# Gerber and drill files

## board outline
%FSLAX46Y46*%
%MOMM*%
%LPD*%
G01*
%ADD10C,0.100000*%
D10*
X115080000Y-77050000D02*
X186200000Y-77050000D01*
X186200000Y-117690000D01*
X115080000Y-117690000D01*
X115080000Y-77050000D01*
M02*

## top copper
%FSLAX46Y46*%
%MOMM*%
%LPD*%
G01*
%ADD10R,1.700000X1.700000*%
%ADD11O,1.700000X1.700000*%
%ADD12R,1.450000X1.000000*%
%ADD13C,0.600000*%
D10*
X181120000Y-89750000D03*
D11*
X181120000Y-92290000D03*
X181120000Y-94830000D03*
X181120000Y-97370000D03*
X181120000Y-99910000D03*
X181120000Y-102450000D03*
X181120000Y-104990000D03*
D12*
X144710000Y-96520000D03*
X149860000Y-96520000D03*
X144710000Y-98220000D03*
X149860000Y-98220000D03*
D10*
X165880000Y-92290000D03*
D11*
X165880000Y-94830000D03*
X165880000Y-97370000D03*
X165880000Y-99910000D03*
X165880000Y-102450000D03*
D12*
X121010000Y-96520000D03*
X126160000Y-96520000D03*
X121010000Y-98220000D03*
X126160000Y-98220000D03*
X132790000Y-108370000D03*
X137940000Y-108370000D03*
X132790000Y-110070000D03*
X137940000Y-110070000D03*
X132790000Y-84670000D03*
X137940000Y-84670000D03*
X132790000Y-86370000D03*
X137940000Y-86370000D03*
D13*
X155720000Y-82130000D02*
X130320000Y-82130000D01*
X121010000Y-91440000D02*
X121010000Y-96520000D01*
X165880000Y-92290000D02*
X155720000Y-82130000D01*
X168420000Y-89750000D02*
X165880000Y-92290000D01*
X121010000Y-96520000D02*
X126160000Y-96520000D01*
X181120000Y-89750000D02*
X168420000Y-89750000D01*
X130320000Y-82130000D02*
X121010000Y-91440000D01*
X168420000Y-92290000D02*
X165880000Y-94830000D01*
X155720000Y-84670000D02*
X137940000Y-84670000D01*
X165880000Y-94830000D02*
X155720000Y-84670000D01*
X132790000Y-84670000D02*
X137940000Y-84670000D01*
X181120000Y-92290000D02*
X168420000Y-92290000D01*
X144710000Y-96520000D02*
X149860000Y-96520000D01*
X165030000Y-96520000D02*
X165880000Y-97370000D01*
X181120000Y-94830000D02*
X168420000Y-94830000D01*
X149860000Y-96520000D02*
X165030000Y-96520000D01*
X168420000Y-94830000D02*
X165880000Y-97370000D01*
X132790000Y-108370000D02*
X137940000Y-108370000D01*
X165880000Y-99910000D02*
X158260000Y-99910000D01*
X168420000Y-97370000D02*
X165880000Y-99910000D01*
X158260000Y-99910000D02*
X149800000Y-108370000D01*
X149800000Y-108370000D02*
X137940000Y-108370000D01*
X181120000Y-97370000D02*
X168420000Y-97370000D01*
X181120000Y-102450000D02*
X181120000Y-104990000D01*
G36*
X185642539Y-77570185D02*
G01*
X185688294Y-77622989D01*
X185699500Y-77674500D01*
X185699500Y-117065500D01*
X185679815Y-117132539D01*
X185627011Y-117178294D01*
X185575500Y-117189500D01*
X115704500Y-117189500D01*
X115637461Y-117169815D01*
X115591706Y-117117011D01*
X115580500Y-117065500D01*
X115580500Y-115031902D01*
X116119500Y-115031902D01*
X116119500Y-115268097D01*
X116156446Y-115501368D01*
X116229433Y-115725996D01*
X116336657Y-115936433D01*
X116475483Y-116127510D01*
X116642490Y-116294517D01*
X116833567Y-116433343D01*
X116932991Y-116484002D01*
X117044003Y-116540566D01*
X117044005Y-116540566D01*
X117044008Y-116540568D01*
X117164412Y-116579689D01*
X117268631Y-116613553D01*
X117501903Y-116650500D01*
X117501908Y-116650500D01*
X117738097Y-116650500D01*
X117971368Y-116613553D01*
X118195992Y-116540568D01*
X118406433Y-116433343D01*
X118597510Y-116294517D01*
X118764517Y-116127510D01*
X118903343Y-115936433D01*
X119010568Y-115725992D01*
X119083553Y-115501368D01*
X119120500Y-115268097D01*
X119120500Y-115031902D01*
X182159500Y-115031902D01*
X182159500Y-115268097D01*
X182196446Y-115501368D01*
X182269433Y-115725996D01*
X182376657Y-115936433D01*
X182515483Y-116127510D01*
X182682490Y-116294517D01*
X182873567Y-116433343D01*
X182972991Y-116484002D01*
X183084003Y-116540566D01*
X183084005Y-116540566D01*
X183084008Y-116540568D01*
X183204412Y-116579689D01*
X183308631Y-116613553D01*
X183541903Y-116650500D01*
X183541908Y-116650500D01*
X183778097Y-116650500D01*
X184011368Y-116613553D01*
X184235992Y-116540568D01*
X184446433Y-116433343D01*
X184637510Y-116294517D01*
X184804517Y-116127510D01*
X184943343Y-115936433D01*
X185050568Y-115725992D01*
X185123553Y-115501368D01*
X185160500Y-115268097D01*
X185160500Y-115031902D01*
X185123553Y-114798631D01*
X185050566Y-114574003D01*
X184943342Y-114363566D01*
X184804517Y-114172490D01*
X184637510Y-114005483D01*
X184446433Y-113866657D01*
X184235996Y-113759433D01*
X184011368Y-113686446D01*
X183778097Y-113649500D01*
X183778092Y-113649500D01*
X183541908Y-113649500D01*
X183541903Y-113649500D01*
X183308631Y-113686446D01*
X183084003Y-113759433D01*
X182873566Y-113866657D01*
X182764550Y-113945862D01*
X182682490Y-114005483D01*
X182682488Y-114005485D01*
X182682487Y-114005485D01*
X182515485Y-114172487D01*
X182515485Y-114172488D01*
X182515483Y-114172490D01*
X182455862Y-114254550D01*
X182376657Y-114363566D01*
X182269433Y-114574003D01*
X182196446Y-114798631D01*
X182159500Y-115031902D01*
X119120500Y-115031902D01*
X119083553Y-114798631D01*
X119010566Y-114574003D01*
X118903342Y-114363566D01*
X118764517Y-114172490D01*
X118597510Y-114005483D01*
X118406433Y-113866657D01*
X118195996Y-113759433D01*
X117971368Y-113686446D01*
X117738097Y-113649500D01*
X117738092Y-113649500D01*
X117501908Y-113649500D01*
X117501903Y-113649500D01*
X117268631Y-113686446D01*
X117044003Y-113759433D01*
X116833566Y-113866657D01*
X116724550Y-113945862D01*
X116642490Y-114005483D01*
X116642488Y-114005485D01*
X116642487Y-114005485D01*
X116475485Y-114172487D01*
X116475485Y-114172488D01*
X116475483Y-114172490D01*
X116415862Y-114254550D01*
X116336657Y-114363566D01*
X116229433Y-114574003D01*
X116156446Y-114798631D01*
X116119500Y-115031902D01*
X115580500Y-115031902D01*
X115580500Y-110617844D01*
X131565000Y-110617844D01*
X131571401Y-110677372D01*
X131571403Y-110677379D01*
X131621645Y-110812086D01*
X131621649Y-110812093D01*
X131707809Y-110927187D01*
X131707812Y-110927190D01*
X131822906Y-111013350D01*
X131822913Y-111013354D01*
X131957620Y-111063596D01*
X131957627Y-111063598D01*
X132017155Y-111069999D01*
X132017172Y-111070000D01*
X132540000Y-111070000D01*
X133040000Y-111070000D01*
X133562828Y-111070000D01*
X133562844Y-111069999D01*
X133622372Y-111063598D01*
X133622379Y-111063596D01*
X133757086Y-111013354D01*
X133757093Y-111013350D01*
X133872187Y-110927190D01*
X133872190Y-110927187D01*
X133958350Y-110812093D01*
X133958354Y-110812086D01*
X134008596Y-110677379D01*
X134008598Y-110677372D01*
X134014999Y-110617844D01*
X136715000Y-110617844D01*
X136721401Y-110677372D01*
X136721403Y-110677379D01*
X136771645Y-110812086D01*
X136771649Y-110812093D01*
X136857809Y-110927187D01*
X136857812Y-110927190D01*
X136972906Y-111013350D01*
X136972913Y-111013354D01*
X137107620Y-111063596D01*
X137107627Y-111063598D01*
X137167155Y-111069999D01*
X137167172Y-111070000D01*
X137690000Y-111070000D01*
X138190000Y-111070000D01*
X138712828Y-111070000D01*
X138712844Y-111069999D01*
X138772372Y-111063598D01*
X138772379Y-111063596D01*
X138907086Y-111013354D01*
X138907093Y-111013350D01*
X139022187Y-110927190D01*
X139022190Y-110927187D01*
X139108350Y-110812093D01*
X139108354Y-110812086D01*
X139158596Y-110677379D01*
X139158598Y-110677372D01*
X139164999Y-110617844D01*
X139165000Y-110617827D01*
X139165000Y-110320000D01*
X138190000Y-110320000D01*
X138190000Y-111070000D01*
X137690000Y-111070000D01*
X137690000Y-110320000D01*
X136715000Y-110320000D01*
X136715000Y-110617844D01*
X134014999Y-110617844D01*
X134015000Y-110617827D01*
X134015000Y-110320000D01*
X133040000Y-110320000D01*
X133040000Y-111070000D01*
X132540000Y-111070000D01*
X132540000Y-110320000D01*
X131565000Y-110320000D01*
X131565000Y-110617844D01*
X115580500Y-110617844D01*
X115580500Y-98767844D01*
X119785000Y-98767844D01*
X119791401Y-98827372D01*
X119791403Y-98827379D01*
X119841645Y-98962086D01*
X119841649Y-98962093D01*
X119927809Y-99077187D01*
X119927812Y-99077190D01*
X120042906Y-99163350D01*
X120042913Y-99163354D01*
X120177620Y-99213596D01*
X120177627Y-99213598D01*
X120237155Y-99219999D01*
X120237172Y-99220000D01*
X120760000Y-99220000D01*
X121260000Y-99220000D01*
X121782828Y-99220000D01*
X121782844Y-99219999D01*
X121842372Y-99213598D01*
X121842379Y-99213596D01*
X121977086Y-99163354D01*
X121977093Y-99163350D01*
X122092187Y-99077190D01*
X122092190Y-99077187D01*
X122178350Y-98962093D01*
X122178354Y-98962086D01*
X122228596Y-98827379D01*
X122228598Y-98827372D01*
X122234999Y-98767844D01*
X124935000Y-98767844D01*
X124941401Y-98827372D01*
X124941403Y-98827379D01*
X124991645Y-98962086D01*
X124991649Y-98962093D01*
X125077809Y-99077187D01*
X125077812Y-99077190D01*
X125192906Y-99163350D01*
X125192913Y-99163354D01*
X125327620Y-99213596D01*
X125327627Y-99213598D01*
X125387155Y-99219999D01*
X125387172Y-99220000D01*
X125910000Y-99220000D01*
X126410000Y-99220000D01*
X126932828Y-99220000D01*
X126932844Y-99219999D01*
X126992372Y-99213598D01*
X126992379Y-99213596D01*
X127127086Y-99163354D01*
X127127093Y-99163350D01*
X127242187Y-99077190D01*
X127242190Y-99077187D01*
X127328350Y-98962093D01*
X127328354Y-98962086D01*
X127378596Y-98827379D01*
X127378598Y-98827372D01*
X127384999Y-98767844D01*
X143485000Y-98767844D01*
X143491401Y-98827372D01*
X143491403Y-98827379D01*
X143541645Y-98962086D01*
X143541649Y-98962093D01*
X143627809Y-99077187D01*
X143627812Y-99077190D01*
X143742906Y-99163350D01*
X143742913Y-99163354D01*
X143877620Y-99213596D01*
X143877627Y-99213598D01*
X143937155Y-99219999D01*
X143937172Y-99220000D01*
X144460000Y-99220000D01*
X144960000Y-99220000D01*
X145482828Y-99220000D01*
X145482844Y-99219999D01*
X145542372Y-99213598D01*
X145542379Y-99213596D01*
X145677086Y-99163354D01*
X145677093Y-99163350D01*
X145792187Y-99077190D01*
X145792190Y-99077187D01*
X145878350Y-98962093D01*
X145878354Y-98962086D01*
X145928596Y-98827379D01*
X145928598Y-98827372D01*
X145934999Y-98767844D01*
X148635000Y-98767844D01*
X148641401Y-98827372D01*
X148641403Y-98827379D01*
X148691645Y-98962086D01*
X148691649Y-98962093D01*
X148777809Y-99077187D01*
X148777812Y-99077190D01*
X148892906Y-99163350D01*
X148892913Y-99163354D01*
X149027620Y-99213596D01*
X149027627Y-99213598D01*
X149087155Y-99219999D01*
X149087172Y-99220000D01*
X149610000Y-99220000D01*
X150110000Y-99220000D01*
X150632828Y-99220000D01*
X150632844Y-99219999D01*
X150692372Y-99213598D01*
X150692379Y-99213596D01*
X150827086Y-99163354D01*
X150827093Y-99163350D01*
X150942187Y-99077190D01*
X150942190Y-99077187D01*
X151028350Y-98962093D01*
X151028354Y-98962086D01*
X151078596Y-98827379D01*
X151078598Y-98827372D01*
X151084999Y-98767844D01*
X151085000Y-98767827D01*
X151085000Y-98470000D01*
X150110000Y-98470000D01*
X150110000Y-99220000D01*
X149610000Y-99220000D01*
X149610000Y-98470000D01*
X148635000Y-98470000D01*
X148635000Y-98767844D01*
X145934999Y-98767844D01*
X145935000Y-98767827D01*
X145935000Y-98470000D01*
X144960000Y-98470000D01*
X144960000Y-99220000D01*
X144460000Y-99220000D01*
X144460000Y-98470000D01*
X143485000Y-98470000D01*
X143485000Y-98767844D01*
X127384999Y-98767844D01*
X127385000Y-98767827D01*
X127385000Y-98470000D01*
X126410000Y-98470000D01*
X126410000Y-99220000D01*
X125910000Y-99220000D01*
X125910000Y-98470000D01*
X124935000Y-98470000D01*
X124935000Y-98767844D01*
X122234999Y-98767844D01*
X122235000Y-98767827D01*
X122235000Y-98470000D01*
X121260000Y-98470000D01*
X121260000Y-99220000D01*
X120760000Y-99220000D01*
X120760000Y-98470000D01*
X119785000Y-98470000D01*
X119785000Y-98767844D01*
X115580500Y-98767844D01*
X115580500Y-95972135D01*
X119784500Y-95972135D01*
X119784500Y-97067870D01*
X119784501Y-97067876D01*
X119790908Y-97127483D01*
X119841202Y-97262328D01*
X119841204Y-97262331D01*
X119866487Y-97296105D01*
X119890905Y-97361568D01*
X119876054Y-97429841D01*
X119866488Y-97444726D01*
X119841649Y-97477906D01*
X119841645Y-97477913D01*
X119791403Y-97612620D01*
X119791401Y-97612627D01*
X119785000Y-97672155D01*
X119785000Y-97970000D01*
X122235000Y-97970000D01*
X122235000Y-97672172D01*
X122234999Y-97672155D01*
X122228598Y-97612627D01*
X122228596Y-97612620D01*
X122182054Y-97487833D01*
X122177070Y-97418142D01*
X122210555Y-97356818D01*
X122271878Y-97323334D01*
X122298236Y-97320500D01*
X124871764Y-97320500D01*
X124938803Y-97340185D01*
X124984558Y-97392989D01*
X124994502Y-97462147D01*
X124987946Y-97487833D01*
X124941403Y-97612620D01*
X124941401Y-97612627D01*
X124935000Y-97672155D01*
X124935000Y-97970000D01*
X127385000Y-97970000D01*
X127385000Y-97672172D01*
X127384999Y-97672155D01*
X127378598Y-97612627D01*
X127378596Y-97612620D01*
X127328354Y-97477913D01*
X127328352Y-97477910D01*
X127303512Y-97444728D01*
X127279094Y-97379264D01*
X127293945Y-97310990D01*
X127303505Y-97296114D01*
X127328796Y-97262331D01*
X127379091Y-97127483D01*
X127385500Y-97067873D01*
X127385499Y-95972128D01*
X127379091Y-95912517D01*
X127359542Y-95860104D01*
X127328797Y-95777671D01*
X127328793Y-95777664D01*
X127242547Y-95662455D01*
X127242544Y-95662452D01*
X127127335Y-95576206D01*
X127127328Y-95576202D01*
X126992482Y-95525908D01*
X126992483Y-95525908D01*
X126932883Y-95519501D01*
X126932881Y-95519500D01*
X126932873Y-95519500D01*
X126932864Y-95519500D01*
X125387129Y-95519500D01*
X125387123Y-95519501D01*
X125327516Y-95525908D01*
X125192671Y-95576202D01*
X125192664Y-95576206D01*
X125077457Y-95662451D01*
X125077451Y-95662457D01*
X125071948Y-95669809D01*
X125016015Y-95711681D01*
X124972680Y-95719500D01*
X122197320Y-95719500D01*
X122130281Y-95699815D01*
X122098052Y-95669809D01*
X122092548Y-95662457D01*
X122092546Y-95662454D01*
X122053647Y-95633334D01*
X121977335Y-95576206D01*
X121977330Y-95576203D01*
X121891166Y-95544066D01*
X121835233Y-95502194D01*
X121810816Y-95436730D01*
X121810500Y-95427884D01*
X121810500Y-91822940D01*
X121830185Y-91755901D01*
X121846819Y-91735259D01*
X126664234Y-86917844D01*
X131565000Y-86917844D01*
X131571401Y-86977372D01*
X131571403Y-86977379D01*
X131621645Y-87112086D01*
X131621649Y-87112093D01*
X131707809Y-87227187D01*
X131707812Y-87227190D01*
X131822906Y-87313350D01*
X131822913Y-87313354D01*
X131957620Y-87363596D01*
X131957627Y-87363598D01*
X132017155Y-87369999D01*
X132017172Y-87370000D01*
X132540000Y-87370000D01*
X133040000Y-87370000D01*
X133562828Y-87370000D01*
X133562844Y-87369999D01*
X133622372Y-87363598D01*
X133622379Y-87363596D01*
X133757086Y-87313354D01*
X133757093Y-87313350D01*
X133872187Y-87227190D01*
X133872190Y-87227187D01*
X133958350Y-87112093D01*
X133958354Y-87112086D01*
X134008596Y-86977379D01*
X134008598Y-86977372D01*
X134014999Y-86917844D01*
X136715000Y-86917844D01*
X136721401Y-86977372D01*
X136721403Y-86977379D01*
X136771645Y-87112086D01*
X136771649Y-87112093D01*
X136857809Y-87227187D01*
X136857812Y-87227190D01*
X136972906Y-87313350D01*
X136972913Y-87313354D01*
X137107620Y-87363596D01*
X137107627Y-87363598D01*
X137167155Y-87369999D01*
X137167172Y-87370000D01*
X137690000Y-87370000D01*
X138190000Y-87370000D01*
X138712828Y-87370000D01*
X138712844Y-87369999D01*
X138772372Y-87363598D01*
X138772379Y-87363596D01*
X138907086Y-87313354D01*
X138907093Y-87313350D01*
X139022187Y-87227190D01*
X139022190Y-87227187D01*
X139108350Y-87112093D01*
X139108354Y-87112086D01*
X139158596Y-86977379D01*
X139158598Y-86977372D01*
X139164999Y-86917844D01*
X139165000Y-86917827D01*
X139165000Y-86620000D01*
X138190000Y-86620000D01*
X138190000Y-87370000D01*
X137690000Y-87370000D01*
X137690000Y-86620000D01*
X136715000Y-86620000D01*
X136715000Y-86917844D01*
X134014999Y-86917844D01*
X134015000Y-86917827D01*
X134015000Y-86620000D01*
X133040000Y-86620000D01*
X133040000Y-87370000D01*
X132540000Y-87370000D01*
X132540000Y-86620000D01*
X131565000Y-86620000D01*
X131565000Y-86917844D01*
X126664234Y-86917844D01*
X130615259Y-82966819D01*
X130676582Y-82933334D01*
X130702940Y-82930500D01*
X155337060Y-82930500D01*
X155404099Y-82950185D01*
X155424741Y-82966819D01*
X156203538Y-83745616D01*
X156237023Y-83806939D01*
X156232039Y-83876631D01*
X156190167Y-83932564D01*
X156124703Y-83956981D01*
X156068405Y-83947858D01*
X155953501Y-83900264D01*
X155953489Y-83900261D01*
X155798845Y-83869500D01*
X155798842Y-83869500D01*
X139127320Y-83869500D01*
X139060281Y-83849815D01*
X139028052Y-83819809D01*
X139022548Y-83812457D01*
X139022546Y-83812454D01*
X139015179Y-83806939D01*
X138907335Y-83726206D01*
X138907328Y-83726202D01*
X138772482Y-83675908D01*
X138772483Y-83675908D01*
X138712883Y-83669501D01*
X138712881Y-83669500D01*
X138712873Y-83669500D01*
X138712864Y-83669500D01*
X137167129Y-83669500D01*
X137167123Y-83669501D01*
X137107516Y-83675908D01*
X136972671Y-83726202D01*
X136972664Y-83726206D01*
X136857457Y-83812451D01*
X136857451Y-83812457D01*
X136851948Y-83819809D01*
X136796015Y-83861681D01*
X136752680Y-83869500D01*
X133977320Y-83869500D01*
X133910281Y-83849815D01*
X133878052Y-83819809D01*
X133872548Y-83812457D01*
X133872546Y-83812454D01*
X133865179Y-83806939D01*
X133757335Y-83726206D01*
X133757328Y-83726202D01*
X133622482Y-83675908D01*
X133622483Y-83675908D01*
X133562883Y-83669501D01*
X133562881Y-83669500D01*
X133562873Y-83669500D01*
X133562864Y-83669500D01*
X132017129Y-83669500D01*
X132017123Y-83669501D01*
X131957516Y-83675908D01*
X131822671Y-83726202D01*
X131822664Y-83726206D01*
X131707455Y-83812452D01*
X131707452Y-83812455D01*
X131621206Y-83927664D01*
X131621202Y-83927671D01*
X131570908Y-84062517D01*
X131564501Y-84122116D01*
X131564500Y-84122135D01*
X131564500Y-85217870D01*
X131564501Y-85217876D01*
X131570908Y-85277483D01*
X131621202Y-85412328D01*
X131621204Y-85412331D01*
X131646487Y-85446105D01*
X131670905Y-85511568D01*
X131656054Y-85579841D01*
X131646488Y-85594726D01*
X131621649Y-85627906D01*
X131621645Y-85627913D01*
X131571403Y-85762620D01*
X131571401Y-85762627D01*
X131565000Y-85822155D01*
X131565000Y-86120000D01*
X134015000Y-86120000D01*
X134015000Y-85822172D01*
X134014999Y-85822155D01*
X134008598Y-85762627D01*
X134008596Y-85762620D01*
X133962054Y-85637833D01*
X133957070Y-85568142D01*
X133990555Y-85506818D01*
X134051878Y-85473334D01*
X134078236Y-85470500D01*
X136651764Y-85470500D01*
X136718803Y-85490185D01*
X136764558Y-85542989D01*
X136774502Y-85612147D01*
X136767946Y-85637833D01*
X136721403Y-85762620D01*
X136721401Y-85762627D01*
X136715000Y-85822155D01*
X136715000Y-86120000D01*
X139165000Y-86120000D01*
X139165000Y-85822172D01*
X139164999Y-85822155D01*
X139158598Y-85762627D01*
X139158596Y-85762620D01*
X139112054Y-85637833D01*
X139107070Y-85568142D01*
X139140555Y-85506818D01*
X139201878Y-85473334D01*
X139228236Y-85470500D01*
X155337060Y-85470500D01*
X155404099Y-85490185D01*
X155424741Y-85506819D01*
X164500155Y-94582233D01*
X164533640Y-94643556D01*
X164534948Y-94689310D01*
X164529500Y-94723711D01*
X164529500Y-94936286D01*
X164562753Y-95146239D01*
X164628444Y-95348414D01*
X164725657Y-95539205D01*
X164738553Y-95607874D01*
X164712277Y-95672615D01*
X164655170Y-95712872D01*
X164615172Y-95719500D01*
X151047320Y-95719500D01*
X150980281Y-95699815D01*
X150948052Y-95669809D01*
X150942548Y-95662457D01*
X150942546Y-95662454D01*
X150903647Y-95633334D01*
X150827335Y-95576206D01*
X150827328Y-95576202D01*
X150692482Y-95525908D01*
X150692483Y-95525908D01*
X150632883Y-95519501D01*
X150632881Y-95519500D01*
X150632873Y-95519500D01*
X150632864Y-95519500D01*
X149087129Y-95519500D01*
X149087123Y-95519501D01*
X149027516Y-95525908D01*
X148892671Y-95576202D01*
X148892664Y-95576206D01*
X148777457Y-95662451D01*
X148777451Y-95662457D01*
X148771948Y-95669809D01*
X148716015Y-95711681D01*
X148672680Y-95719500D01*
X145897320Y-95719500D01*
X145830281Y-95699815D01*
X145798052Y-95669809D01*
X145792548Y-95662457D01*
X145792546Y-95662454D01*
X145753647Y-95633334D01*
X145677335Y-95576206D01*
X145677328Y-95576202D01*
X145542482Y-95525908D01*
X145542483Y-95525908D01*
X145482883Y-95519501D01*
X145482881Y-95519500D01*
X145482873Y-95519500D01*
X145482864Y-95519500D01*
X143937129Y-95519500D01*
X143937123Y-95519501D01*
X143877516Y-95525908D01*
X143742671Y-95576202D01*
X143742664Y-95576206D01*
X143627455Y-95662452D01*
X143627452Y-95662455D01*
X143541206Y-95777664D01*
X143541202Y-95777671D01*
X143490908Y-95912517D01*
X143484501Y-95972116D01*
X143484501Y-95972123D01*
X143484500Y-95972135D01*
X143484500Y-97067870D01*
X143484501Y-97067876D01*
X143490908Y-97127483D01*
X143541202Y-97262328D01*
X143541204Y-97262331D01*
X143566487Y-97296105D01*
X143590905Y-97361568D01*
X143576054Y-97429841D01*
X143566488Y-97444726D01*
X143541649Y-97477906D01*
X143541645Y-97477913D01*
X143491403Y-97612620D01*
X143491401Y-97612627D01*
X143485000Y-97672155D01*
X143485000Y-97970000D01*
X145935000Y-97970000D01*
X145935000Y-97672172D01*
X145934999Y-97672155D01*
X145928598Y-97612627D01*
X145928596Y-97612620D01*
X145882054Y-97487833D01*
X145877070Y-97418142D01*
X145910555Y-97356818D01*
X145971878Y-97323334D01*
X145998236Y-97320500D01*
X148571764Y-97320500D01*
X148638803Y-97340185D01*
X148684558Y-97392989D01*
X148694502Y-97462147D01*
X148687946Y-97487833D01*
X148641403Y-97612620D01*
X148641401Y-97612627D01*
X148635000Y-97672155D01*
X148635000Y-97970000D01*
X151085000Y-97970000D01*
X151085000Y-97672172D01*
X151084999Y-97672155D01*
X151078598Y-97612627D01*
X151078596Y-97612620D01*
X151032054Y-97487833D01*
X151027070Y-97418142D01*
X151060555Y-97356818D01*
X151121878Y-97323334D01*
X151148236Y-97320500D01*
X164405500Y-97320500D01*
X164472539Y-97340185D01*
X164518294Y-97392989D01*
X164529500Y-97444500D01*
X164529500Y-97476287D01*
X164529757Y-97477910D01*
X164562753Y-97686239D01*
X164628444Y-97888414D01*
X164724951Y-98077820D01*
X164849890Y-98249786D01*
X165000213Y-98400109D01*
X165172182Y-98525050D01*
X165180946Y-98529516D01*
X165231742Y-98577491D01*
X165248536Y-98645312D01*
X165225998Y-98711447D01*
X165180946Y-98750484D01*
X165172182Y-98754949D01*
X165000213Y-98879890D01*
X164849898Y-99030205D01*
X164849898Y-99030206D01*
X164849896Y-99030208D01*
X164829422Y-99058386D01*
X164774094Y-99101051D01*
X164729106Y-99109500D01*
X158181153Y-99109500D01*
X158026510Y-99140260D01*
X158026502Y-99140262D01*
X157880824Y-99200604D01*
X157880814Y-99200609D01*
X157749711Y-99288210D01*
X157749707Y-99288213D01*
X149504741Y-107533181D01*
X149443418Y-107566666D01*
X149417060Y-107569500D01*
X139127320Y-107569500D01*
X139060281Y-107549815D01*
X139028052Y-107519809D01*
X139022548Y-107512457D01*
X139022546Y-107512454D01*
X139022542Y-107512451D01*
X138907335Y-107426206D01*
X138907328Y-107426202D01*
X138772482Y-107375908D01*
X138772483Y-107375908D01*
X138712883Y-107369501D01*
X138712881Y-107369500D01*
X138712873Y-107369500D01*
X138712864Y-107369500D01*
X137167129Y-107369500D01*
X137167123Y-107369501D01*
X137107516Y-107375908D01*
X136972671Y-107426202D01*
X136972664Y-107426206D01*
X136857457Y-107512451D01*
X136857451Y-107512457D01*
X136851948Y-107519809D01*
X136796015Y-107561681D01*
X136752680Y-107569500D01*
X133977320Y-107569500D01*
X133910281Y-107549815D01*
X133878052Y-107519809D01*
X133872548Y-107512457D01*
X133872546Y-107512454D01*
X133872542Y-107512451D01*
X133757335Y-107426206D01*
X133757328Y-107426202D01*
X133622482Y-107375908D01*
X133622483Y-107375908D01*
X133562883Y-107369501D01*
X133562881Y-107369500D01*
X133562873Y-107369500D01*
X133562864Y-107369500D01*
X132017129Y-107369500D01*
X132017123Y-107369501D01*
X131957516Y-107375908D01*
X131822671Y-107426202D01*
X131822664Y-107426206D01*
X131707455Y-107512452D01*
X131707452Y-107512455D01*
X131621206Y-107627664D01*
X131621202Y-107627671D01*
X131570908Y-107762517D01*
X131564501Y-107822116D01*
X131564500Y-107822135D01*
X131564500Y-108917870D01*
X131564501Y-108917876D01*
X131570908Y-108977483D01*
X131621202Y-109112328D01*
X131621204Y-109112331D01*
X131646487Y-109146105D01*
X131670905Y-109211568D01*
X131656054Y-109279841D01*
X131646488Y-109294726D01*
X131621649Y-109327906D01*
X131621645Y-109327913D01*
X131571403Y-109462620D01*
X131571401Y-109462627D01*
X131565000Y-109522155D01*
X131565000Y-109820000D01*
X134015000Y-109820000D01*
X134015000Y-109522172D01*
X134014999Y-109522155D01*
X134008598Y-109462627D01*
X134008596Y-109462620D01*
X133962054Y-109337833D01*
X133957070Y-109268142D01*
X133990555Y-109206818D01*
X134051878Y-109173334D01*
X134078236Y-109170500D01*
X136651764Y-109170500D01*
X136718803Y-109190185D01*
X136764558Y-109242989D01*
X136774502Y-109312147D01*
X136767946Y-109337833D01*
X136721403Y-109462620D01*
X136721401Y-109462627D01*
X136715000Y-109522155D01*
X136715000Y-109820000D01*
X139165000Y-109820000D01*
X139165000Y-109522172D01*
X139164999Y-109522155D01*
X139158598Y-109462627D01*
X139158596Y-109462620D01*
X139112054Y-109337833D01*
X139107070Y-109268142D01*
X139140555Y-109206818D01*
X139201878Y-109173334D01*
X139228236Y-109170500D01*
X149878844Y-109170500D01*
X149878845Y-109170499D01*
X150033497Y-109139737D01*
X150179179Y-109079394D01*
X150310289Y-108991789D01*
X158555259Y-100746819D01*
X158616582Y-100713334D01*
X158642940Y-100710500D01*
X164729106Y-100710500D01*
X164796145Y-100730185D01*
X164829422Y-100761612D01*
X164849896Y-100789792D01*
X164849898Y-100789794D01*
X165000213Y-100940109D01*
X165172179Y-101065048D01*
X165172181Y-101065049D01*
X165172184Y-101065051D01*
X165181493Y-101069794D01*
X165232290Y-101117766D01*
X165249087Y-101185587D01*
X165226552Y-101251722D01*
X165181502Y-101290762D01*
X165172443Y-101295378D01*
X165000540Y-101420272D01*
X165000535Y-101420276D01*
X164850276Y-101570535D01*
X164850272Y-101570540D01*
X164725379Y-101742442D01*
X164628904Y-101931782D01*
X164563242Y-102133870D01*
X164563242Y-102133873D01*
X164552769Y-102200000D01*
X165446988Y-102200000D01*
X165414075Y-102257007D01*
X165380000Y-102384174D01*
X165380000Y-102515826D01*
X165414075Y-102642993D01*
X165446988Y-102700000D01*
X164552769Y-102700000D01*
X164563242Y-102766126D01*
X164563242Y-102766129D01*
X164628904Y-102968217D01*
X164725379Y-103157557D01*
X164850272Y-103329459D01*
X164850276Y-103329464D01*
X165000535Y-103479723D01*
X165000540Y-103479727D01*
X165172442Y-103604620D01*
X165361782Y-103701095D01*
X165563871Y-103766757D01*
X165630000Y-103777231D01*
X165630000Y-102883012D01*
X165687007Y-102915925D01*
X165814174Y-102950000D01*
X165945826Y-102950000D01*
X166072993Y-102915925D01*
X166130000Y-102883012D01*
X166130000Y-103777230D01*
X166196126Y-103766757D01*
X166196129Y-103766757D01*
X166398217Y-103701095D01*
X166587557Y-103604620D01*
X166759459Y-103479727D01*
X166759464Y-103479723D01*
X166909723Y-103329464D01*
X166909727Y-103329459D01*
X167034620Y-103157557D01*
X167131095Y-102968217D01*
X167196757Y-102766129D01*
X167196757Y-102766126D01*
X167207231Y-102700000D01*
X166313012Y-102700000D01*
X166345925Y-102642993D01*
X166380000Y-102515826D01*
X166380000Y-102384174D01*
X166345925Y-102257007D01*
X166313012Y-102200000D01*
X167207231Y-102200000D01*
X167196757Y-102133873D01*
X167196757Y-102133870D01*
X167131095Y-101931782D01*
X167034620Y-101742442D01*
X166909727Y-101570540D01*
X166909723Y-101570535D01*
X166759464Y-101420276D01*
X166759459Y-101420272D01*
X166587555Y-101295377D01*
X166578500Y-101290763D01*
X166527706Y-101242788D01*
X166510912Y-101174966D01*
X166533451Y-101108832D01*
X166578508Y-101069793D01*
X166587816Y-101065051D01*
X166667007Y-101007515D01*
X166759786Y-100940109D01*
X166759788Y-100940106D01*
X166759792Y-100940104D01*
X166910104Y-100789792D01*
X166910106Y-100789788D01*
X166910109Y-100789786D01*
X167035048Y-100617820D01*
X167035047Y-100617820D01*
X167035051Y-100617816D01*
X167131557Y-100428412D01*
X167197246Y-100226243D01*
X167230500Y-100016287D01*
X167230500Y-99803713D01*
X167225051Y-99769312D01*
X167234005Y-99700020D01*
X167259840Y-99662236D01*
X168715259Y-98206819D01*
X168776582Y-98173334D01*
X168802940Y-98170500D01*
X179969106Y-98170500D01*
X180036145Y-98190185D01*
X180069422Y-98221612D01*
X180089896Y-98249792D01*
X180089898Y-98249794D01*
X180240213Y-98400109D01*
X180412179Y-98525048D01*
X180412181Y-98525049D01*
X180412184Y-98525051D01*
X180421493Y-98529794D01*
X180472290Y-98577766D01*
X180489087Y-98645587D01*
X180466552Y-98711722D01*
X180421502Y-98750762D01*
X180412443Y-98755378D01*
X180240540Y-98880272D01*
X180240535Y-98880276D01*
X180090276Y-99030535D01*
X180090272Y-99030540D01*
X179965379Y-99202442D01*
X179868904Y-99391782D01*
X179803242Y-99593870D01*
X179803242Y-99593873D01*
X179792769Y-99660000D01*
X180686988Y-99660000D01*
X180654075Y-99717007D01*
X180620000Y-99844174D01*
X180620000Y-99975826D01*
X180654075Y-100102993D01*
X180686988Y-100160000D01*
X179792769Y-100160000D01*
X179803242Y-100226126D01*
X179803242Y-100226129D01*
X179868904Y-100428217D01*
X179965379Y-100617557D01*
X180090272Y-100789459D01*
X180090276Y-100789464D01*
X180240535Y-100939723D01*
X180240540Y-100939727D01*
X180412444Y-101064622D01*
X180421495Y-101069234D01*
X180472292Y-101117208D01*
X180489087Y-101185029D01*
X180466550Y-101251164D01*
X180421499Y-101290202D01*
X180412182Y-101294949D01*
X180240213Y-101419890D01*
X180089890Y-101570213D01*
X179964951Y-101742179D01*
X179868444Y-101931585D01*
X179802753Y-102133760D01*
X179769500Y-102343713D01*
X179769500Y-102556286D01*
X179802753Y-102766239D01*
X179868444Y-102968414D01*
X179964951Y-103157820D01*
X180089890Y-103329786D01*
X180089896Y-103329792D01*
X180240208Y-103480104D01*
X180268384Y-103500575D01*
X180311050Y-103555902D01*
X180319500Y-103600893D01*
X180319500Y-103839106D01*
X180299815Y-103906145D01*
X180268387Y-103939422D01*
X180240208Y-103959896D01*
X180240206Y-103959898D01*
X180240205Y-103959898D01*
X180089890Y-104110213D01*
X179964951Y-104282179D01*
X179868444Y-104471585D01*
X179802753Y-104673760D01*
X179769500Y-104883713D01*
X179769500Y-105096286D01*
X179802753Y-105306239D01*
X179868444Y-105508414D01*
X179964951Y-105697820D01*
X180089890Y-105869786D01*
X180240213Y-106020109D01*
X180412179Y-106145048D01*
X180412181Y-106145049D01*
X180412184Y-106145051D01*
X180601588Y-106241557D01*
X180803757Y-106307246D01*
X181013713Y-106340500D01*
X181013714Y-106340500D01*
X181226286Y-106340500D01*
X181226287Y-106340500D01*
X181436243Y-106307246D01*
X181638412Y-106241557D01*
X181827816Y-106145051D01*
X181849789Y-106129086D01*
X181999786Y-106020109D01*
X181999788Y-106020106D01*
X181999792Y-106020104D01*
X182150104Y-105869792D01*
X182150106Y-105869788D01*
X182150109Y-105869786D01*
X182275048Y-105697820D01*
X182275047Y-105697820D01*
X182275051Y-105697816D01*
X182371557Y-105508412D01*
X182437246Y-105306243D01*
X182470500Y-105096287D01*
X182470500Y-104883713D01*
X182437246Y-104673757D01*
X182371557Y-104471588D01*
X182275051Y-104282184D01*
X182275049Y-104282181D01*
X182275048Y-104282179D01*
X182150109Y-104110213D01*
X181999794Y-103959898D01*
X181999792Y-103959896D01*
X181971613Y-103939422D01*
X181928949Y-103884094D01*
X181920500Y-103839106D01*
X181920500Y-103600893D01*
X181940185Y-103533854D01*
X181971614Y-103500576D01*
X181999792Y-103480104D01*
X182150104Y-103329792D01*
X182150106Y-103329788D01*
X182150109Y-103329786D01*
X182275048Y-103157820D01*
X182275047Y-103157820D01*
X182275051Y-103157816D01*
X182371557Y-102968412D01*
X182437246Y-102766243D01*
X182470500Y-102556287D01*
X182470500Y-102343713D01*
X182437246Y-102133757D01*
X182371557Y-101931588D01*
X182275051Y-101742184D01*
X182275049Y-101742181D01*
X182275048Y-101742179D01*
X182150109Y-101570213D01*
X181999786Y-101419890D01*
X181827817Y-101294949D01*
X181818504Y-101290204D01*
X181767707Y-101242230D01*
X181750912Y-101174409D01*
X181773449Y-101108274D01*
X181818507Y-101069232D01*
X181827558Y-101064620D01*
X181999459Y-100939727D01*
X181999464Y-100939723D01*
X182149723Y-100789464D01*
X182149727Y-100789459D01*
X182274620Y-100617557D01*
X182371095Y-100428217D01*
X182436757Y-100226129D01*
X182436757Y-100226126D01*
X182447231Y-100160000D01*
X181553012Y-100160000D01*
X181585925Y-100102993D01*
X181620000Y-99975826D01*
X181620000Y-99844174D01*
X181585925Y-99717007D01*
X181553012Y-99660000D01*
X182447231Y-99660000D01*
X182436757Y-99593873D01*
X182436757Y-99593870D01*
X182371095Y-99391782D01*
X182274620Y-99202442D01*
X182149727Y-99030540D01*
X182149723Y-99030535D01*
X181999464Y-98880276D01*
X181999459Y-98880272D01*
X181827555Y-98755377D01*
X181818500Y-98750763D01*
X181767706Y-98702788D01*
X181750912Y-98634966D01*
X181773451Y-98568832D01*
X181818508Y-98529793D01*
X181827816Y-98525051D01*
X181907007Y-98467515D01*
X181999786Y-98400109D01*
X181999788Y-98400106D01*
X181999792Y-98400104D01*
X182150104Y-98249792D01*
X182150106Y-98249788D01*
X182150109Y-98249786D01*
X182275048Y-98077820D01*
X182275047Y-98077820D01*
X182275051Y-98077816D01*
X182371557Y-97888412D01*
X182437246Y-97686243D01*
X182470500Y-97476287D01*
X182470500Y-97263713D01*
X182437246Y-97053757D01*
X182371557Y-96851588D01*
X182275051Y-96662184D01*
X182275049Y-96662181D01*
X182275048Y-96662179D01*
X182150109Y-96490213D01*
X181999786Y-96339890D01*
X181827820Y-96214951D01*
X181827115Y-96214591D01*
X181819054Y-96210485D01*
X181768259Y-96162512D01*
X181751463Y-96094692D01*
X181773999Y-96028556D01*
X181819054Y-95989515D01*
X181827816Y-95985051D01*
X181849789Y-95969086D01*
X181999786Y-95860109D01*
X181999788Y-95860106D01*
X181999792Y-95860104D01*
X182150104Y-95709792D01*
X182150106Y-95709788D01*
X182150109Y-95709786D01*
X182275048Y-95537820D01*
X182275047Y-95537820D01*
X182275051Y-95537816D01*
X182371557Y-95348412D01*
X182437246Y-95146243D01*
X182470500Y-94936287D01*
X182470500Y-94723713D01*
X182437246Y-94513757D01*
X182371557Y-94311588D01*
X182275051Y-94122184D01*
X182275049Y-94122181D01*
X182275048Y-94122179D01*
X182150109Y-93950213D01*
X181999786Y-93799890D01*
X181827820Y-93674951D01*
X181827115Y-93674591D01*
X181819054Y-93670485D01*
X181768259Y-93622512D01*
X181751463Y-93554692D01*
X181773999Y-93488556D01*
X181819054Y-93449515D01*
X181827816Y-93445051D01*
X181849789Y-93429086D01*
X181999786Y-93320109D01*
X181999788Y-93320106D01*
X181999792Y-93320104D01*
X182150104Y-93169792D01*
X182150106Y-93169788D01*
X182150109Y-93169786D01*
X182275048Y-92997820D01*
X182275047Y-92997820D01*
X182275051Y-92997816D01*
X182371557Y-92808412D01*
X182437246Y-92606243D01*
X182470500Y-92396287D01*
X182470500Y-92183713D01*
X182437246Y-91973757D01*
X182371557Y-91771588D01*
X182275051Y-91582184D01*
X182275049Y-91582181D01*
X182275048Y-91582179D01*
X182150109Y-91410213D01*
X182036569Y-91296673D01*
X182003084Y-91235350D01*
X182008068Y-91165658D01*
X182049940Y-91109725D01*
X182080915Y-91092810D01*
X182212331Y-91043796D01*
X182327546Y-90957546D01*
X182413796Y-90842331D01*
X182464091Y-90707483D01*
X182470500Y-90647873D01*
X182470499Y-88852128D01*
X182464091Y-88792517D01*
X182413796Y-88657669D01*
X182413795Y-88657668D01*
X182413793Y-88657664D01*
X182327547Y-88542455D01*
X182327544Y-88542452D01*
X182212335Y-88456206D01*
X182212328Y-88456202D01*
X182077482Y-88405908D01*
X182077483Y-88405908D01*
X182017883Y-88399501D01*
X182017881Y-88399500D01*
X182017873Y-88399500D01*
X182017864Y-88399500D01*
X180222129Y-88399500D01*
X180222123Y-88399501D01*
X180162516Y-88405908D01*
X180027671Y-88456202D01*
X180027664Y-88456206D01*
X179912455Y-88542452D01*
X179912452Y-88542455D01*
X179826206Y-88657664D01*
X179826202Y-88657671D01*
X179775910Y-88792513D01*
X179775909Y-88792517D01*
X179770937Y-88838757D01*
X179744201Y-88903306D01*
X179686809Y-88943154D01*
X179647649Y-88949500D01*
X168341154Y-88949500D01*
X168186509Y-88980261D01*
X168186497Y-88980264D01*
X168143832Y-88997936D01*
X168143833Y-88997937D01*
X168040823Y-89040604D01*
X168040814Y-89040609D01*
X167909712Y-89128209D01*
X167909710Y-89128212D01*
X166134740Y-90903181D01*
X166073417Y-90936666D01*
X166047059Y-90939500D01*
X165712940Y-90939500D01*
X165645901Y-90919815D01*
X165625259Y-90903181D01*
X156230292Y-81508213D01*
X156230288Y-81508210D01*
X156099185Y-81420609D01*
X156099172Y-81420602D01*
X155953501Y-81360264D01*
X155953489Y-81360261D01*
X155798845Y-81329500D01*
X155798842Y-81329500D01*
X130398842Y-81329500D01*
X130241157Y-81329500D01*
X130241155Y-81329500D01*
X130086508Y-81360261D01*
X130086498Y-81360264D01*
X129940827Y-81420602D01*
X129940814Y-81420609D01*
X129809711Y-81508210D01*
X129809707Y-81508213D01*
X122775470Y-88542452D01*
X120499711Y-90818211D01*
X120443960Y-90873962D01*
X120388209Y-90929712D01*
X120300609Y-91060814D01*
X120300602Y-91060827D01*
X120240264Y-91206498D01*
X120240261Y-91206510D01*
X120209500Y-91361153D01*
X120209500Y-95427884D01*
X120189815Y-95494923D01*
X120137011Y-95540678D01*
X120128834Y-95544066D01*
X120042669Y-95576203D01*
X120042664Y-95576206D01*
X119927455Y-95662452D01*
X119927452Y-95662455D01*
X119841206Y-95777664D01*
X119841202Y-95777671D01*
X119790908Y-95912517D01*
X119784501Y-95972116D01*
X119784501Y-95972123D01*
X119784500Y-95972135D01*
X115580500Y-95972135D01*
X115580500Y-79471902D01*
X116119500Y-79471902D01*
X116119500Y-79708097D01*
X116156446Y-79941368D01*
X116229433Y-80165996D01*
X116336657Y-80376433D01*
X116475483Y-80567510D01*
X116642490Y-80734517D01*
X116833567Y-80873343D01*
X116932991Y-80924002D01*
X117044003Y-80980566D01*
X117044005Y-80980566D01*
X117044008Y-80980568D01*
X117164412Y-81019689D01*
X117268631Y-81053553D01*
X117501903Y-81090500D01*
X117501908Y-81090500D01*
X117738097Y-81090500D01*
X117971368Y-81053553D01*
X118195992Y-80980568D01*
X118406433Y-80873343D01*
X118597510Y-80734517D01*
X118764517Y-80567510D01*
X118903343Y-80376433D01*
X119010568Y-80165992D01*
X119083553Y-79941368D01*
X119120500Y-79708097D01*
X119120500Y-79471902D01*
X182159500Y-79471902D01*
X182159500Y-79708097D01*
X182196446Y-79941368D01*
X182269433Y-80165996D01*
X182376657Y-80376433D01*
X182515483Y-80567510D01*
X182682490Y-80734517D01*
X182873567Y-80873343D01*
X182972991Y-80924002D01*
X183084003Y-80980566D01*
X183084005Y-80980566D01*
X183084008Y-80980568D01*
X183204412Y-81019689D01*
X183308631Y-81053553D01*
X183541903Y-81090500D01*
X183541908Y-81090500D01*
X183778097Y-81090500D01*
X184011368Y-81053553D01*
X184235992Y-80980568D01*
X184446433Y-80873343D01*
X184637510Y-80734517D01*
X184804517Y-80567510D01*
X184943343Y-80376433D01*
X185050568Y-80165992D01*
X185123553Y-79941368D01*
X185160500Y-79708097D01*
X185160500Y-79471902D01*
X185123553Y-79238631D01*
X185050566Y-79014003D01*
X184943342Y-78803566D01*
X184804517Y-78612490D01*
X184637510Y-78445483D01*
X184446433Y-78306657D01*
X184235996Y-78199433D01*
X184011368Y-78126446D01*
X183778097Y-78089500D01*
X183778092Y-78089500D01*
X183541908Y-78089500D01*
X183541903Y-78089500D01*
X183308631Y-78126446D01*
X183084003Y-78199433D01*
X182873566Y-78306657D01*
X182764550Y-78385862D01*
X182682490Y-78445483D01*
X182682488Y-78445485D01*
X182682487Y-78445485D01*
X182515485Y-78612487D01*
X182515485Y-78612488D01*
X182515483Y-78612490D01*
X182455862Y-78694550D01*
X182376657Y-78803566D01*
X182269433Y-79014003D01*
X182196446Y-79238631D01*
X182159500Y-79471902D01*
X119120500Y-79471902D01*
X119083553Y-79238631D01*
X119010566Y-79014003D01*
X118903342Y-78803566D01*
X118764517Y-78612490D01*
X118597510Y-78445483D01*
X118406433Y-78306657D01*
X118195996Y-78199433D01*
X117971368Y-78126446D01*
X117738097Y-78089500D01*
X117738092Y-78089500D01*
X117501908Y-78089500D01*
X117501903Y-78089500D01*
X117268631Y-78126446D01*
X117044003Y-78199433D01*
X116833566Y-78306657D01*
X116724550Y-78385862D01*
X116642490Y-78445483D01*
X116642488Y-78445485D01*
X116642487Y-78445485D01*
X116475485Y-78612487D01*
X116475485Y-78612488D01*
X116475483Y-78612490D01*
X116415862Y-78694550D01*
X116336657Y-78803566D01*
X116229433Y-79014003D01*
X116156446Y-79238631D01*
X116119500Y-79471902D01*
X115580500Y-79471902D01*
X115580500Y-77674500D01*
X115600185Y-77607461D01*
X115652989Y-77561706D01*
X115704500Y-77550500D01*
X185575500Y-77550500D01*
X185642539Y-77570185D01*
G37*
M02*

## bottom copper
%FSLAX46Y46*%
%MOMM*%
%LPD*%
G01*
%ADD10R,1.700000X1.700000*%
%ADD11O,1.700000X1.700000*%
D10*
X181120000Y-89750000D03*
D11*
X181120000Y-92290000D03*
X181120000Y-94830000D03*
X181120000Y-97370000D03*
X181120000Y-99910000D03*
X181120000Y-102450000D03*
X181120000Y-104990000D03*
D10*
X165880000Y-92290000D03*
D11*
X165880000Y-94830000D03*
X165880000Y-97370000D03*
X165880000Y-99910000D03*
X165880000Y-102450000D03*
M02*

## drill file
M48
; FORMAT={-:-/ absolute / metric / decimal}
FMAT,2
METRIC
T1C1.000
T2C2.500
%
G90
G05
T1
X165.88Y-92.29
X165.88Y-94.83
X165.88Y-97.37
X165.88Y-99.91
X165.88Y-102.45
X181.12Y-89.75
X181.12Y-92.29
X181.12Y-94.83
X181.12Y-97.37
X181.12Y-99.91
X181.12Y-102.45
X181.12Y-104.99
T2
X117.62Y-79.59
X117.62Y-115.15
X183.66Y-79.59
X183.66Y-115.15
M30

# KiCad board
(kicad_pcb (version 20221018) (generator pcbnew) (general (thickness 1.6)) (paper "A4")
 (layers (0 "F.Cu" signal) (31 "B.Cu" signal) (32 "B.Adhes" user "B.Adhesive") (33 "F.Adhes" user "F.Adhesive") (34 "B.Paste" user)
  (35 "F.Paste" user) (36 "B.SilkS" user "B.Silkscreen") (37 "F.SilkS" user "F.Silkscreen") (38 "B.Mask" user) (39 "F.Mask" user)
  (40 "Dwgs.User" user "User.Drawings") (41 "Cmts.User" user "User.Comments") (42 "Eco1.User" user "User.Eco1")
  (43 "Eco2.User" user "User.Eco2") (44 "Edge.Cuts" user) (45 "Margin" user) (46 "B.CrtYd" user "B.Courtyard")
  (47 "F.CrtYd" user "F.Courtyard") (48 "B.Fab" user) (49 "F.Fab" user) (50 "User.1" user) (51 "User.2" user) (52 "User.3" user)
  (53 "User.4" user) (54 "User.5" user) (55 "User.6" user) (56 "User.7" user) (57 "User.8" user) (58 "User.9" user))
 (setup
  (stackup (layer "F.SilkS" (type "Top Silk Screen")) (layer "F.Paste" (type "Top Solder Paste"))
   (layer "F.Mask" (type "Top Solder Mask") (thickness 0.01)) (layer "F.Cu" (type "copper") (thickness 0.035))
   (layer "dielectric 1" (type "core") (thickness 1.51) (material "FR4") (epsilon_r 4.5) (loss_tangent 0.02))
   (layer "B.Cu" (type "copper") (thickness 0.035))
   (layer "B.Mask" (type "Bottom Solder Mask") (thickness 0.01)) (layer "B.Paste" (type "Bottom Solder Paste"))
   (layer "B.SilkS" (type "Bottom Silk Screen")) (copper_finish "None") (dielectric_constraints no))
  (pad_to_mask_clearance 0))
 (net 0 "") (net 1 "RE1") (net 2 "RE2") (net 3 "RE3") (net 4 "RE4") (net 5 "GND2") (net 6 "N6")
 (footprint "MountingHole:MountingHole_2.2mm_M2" (layer "F.Cu") (at 117.62 115.15)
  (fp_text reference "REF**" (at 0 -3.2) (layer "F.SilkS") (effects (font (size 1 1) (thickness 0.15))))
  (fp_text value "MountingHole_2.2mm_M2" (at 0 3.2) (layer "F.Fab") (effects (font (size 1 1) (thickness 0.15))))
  (pad "" np_thru_hole circle (at 0 0) (size 2.5 2.5) (drill 2.5) (layers "F&B.Cu" "*.Mask")))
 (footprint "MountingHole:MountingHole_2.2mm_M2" (layer "F.Cu") (at 183.66 79.59)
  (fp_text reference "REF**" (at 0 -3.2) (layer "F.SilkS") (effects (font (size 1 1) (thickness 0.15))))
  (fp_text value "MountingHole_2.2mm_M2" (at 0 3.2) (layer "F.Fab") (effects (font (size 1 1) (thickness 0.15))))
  (pad "" np_thru_hole circle (at 0 0) (size 2.5 2.5) (drill 2.5) (layers "F&B.Cu" "*.Mask")))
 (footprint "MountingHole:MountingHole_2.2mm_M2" (layer "F.Cu") (at 183.66 115.15)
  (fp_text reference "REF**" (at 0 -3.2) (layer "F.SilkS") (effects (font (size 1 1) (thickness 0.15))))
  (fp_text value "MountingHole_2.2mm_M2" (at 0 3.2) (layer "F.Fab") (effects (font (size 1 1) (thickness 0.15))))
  (pad "" np_thru_hole circle (at 0 0) (size 2.5 2.5) (drill 2.5) (layers "F&B.Cu" "*.Mask")))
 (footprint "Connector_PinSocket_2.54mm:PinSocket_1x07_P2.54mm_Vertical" (layer "F.Cu") (at 181.12 89.75)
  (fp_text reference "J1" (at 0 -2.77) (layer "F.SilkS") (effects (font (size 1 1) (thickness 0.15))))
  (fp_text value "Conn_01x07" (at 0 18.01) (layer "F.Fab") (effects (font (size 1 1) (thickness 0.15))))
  (pad "1" thru_hole rect (at 0 0) (size 1.7 1.7) (drill 1) (layers "*.Cu" "*.Mask") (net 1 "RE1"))
  (pad "2" thru_hole oval (at 0 2.54) (size 1.7 1.7) (drill 1) (layers "*.Cu" "*.Mask") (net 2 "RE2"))
  (pad "3" thru_hole oval (at 0 5.08) (size 1.7 1.7) (drill 1) (layers "*.Cu" "*.Mask") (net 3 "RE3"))
  (pad "4" thru_hole oval (at 0 7.62) (size 1.7 1.7) (drill 1) (layers "*.Cu" "*.Mask") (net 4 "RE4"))
  (pad "5" thru_hole oval (at 0 10.16) (size 1.7 1.7) (drill 1) (layers "*.Cu" "*.Mask") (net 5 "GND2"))
  (pad "6" thru_hole oval (at 0 12.7) (size 1.7 1.7) (drill 1) (layers "*.Cu" "*.Mask") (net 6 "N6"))
  (pad "7" thru_hole oval (at 0 15.24) (size 1.7 1.7) (drill 1) (layers "*.Cu" "*.Mask") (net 6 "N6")))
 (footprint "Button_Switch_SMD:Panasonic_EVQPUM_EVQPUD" (layer "F.Cu") (at 147.285 97.37)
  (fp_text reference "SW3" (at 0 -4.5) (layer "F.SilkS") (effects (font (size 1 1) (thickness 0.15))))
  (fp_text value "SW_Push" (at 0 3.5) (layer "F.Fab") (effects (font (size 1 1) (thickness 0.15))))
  (pad "1" smd rect (at -2.575 -0.85 180) (size 1.45 1) (layers "F.Cu" "F.Paste" "F.Mask") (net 3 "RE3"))
  (pad "1" smd rect (at 2.575 -0.85 180) (size 1.45 1) (layers "F.Cu" "F.Paste" "F.Mask") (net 3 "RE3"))
  (pad "2" smd rect (at -2.575 0.85 180) (size 1.45 1) (layers "F.Cu" "F.Paste" "F.Mask") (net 5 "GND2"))
  (pad "2" smd rect (at 2.575 0.85 180) (size 1.45 1) (layers "F.Cu" "F.Paste" "F.Mask") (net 5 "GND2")))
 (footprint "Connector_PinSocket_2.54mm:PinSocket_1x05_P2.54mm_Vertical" (layer "F.Cu") (at 165.88 92.29)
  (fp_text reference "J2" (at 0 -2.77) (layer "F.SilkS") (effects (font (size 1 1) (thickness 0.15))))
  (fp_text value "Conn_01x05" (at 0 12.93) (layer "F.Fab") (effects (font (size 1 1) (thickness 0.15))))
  (pad "1" thru_hole rect (at 0 0) (size 1.7 1.7) (drill 1) (layers "*.Cu" "*.Mask") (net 1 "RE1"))
  (pad "2" thru_hole oval (at 0 2.54) (size 1.7 1.7) (drill 1) (layers "*.Cu" "*.Mask") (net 2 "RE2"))
  (pad "3" thru_hole oval (at 0 5.08) (size 1.7 1.7) (drill 1) (layers "*.Cu" "*.Mask") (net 3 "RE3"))
  (pad "4" thru_hole oval (at 0 7.62) (size 1.7 1.7) (drill 1) (layers "*.Cu" "*.Mask") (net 4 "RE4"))
  (pad "5" thru_hole oval (at 0 10.16) (size 1.7 1.7) (drill 1) (layers "*.Cu" "*.Mask") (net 5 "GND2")))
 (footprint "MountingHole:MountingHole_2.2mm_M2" (layer "F.Cu") (at 117.62 79.59)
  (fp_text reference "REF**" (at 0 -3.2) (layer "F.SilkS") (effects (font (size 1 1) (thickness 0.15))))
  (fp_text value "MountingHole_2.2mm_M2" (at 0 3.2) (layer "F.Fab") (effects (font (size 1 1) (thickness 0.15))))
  (pad "" np_thru_hole circle (at 0 0) (size 2.5 2.5) (drill 2.5) (layers "F&B.Cu" "*.Mask")))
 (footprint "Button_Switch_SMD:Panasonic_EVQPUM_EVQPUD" (layer "F.Cu") (at 123.585 97.37)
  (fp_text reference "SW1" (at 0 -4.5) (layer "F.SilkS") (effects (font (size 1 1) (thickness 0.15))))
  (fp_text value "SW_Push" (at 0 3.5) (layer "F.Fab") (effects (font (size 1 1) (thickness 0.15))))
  (pad "1" smd rect (at -2.575 -0.85 180) (size 1.45 1) (layers "F.Cu" "F.Paste" "F.Mask") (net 1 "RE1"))
  (pad "1" smd rect (at 2.575 -0.85 180) (size 1.45 1) (layers "F.Cu" "F.Paste" "F.Mask") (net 1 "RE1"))
  (pad "2" smd rect (at -2.575 0.85 180) (size 1.45 1) (layers "F.Cu" "F.Paste" "F.Mask") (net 5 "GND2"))
  (pad "2" smd rect (at 2.575 0.85 180) (size 1.45 1) (layers "F.Cu" "F.Paste" "F.Mask") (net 5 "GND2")))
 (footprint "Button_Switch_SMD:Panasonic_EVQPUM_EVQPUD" (layer "F.Cu") (at 135.365 109.22)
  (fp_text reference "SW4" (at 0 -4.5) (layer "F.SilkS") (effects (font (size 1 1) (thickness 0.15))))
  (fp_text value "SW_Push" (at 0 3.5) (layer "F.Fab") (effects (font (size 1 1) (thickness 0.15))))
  (pad "1" smd rect (at -2.575 -0.85 180) (size 1.45 1) (layers "F.Cu" "F.Paste" "F.Mask") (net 4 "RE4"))
  (pad "1" smd rect (at 2.575 -0.85 180) (size 1.45 1) (layers "F.Cu" "F.Paste" "F.Mask") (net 4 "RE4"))
  (pad "2" smd rect (at -2.575 0.85 180) (size 1.45 1) (layers "F.Cu" "F.Paste" "F.Mask") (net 5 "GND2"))
  (pad "2" smd rect (at 2.575 0.85 180) (size 1.45 1) (layers "F.Cu" "F.Paste" "F.Mask") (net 5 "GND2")))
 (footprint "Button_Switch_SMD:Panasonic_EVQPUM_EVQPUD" (layer "F.Cu") (at 135.365 85.52)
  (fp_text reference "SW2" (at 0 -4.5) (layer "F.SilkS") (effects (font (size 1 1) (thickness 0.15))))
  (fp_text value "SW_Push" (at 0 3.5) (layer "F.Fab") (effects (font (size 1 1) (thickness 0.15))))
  (pad "1" smd rect (at -2.575 -0.85 180) (size 1.45 1) (layers "F.Cu" "F.Paste" "F.Mask") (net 2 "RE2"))
  (pad "1" smd rect (at 2.575 -0.85 180) (size 1.45 1) (layers "F.Cu" "F.Paste" "F.Mask") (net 2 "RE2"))
  (pad "2" smd rect (at -2.575 0.85 180) (size 1.45 1) (layers "F.Cu" "F.Paste" "F.Mask") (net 5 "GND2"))
  (pad "2" smd rect (at 2.575 0.85 180) (size 1.45 1) (layers "F.Cu" "F.Paste" "F.Mask") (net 5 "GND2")))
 (gr_rect (start 115.08 77.05) (end 186.2 117.69) (stroke (width 0.1) (type default)) (fill none) (layer "Edge.Cuts"))
 (segment (start 155.72 82.13) (end 130.32 82.13) (width 0.6) (layer "F.Cu") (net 1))
 (segment (start 121.01 91.44) (end 121.01 96.52) (width 0.6) (layer "F.Cu") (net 1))
 (segment (start 165.88 92.29) (end 155.72 82.13) (width 0.6) (layer "F.Cu") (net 1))
 (segment (start 168.42 89.75) (end 165.88 92.29) (width 0.6) (layer "F.Cu") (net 1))
 (segment (start 121.01 96.52) (end 126.16 96.52) (width 0.6) (layer "F.Cu") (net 1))
 (segment (start 181.12 89.75) (end 168.42 89.75) (width 0.6) (layer "F.Cu") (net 1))
 (segment (start 130.32 82.13) (end 121.01 91.44) (width 0.6) (layer "F.Cu") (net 1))
 (segment (start 168.42 92.29) (end 165.88 94.83) (width 0.6) (layer "F.Cu") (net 2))
 (segment (start 155.72 84.67) (end 137.94 84.67) (width 0.6) (layer "F.Cu") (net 2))
 (segment (start 165.88 94.83) (end 155.72 84.67) (width 0.6) (layer "F.Cu") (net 2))
 (segment (start 132.79 84.67) (end 137.94 84.67) (width 0.6) (layer "F.Cu") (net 2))
 (segment (start 181.12 92.29) (end 168.42 92.29) (width 0.6) (layer "F.Cu") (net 2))
 (segment (start 144.71 96.52) (end 149.86 96.52) (width 0.6) (layer "F.Cu") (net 3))
 (segment (start 165.03 96.52) (end 165.88 97.37) (width 0.6) (layer "F.Cu") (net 3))
 (segment (start 181.12 94.83) (end 168.42 94.83) (width 0.6) (layer "F.Cu") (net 3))
 (segment (start 149.86 96.52) (end 165.03 96.52) (width 0.6) (layer "F.Cu") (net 3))
 (segment (start 168.42 94.83) (end 165.88 97.37) (width 0.6) (layer "F.Cu") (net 3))
 (segment (start 132.79 108.37) (end 137.94 108.37) (width 0.6) (layer "F.Cu") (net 4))
 (segment (start 165.88 99.91) (end 158.26 99.91) (width 0.6) (layer "F.Cu") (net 4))
 (segment (start 168.42 97.37) (end 165.88 99.91) (width 0.6) (layer "F.Cu") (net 4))
 (segment (start 158.26 99.91) (end 149.8 108.37) (width 0.6) (layer "F.Cu") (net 4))
 (segment (start 149.8 108.37) (end 137.94 108.37) (width 0.6) (layer "F.Cu") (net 4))
 (segment (start 181.12 97.37) (end 168.42 97.37) (width 0.6) (layer "F.Cu") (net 4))
 (segment (start 181.12 102.45) (end 181.12 104.99) (width 0.6) (layer "F.Cu") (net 6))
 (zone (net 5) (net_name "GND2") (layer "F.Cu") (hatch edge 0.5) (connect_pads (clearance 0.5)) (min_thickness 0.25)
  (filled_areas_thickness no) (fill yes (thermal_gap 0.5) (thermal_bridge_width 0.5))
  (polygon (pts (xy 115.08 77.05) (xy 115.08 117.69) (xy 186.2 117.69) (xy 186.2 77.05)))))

